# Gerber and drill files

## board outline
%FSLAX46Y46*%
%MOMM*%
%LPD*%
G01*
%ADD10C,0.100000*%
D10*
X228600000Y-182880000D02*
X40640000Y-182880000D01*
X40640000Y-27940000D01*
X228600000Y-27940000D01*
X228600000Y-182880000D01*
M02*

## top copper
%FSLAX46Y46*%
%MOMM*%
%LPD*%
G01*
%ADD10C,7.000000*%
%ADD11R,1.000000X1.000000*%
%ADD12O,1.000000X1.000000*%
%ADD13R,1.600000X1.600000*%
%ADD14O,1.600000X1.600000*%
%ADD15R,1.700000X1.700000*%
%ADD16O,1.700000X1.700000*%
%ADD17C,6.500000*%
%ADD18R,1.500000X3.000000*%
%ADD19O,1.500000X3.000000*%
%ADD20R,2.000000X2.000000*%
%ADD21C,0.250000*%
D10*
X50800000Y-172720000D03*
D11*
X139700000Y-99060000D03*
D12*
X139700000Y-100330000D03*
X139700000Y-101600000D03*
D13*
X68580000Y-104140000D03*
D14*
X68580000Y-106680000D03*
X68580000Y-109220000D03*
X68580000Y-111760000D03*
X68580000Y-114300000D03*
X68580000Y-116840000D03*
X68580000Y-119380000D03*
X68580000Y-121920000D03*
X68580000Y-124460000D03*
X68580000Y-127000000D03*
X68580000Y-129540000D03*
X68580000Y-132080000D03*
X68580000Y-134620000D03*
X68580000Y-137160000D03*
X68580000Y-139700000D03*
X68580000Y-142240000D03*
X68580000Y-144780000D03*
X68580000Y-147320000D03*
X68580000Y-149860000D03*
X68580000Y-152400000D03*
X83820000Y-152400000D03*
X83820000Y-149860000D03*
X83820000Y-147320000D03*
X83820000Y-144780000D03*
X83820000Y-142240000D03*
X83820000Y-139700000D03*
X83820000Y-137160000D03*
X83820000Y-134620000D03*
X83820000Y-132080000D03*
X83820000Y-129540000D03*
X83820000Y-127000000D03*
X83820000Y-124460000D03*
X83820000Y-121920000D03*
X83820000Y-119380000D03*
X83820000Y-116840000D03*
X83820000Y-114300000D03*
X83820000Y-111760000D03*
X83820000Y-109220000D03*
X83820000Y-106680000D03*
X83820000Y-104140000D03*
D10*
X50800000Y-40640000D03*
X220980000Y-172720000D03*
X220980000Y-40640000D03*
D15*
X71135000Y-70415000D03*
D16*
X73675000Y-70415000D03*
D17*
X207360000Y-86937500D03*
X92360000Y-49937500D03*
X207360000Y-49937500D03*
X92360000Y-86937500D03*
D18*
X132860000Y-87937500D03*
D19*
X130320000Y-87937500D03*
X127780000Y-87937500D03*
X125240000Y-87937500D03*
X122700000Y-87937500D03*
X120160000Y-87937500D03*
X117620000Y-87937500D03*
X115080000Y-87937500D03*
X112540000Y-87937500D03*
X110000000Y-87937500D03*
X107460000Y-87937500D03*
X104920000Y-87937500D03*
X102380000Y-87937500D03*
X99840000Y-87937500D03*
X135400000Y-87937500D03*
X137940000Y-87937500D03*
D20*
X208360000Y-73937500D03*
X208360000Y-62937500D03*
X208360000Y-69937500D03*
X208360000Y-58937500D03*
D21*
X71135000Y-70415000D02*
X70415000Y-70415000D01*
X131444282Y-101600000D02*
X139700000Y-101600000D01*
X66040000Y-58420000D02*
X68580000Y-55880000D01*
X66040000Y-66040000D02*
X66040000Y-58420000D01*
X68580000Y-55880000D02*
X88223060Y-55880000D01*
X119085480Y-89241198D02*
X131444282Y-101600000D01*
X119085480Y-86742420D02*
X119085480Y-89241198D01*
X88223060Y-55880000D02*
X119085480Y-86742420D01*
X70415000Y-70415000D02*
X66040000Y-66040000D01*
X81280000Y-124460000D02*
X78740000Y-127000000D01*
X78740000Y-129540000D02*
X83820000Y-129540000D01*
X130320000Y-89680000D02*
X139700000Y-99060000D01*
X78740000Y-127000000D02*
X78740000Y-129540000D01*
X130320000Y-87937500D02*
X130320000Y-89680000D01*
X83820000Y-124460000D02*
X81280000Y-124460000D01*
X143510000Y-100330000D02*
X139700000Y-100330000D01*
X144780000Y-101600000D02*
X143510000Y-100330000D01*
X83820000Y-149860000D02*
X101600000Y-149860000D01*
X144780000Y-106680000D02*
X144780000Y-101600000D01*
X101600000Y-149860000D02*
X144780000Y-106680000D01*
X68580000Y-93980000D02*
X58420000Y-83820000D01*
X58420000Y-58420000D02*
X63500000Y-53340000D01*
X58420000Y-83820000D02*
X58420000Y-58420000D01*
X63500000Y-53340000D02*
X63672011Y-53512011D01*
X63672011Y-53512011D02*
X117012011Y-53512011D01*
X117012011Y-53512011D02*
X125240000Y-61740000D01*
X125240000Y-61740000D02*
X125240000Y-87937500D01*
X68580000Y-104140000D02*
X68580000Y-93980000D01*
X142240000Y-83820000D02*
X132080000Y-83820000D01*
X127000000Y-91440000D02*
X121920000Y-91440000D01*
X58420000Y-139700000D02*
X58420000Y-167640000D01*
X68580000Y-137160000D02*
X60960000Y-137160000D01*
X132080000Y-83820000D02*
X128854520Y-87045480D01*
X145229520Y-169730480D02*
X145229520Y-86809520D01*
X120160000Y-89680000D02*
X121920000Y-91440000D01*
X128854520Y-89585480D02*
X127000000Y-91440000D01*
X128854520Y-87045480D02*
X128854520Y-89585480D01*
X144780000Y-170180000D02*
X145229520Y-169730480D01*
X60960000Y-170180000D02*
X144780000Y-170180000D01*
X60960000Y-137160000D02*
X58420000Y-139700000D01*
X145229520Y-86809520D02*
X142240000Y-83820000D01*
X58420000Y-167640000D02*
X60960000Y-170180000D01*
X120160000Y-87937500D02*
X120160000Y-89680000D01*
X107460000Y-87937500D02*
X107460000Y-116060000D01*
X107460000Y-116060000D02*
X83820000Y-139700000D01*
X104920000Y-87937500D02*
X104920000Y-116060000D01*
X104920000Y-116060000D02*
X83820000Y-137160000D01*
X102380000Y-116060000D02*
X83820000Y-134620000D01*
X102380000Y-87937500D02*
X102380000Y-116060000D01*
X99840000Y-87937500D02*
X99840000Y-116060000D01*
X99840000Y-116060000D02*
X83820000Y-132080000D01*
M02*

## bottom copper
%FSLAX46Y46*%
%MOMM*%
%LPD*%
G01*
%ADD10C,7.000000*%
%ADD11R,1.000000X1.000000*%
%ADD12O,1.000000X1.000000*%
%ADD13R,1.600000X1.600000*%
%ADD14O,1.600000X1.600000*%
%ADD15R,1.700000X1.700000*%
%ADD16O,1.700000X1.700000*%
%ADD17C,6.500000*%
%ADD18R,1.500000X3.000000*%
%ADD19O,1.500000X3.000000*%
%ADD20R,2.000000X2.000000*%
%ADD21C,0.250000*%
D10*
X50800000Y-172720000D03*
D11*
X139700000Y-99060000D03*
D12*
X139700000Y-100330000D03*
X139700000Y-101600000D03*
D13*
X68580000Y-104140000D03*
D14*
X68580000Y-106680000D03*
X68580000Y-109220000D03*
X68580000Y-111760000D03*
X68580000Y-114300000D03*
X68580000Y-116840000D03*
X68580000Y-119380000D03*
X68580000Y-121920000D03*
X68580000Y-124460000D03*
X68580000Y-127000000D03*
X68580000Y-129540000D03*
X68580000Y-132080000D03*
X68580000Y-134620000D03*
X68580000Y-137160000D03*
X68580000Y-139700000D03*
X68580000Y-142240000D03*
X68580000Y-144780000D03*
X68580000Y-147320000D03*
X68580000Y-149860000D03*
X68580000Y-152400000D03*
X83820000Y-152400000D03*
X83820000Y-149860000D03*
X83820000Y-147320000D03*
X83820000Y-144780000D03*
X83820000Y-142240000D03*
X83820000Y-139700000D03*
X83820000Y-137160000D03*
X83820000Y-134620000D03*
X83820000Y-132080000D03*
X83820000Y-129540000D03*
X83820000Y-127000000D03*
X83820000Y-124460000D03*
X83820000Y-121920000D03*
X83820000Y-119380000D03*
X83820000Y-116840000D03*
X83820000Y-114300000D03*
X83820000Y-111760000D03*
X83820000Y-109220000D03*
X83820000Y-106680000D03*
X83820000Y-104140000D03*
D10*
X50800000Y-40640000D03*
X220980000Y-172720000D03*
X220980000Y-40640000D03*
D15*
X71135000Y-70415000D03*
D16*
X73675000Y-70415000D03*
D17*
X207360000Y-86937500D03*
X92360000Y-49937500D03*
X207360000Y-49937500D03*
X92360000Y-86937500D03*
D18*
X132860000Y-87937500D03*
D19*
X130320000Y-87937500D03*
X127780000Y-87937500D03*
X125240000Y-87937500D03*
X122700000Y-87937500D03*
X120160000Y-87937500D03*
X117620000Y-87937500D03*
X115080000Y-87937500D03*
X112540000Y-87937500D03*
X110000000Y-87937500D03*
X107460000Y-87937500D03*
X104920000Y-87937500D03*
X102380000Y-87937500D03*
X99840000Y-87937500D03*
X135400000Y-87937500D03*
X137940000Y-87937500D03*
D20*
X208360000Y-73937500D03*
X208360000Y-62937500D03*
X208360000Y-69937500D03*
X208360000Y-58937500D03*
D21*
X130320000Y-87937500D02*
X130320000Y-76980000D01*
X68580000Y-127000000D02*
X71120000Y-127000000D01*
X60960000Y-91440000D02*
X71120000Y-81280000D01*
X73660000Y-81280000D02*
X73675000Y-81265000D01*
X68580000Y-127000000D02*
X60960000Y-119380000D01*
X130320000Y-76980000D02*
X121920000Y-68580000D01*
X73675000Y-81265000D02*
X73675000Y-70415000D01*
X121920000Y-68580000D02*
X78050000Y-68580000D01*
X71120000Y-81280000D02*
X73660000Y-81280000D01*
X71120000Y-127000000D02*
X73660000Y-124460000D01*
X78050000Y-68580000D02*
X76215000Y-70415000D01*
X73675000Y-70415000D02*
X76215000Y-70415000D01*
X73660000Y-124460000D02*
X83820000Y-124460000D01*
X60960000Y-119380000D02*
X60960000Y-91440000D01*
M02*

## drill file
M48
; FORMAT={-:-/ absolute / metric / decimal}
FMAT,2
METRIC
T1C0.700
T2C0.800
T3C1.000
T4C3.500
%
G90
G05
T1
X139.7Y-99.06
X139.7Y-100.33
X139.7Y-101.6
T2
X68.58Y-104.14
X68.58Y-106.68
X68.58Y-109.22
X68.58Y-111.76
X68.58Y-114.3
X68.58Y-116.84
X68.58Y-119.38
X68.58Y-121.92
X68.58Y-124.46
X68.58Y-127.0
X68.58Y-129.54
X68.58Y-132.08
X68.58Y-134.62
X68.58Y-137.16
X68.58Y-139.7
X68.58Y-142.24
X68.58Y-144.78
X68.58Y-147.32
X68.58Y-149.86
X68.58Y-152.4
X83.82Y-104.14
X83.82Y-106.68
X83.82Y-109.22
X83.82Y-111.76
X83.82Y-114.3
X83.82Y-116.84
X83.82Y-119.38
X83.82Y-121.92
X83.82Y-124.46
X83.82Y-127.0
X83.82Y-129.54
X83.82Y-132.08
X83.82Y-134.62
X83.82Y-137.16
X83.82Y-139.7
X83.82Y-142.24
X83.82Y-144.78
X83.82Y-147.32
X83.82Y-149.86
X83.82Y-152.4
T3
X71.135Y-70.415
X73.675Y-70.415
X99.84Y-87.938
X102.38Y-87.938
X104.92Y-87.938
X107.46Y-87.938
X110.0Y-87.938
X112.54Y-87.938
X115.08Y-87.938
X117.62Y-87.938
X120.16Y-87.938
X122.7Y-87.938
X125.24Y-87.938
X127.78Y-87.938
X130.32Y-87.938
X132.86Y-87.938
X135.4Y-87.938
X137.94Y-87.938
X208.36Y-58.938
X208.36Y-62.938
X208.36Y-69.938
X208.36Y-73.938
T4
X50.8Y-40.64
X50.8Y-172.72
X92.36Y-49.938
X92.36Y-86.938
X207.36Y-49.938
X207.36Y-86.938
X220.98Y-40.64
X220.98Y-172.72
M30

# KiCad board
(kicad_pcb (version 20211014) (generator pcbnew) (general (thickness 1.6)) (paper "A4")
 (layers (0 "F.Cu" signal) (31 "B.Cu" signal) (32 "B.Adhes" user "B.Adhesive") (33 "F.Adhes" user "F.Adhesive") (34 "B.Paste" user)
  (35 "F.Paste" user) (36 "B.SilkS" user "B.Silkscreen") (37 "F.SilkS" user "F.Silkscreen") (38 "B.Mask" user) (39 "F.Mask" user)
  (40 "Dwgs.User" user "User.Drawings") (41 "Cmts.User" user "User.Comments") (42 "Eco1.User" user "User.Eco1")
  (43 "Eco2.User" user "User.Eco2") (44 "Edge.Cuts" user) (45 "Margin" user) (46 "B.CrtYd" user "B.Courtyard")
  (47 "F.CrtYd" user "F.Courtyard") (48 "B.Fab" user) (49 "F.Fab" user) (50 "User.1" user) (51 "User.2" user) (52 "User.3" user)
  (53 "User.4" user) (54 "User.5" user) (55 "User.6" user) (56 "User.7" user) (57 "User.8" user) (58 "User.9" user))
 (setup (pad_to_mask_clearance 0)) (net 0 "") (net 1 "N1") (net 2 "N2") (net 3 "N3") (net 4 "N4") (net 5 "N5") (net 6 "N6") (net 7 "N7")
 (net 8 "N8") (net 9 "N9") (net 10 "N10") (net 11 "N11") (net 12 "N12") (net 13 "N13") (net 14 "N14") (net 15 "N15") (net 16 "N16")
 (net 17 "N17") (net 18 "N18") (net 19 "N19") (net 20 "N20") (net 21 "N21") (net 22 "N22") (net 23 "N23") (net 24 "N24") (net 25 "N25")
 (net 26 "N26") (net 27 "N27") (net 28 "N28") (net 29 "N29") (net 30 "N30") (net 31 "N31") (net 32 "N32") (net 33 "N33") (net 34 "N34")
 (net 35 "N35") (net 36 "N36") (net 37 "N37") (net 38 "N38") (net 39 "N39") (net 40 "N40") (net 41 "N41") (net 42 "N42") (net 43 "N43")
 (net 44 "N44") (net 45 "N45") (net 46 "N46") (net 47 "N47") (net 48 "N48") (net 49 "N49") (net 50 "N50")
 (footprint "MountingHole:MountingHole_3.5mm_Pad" (layer "F.Cu") (at 50.8 172.72)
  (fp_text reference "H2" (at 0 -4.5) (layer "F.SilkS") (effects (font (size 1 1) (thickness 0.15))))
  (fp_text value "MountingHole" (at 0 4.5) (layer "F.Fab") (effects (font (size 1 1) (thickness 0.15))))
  (pad "1" thru_hole circle (at 0 0) (size 7 7) (drill 3.5) (layers *.Cu *.Mask)))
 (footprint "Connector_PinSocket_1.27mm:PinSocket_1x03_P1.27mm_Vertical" (layer "F.Cu") (at 139.7 99.06)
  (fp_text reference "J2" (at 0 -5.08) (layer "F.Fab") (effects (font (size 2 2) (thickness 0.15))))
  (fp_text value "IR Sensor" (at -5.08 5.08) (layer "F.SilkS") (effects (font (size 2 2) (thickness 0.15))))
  (pad "1" thru_hole rect (at 0 0) (size 1 1) (drill 0.7) (layers *.Cu *.Mask) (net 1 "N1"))
  (pad "2" thru_hole oval (at 0 1.27) (size 1 1) (drill 0.7) (layers *.Cu *.Mask) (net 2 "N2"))
  (pad "3" thru_hole oval (at 0 2.54) (size 1 1) (drill 0.7) (layers *.Cu *.Mask) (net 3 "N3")))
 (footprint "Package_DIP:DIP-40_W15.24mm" (layer "F.Cu") (at 68.58 104.14)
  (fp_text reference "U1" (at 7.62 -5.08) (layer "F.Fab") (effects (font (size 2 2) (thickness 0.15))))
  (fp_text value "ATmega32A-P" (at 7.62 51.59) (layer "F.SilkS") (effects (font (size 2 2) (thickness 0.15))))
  (pad "1" thru_hole rect (at 0 0) (size 1.6 1.6) (drill 0.8) (layers *.Cu *.Mask) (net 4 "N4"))
  (pad "2" thru_hole oval (at 0 2.54) (size 1.6 1.6) (drill 0.8) (layers *.Cu *.Mask) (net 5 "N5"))
  (pad "3" thru_hole oval (at 0 5.08) (size 1.6 1.6) (drill 0.8) (layers *.Cu *.Mask) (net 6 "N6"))
  (pad "4" thru_hole oval (at 0 7.62) (size 1.6 1.6) (drill 0.8) (layers *.Cu *.Mask) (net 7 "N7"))
  (pad "5" thru_hole oval (at 0 10.16) (size 1.6 1.6) (drill 0.8) (layers *.Cu *.Mask) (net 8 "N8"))
  (pad "6" thru_hole oval (at 0 12.7) (size 1.6 1.6) (drill 0.8) (layers *.Cu *.Mask) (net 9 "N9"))
  (pad "7" thru_hole oval (at 0 15.24) (size 1.6 1.6) (drill 0.8) (layers *.Cu *.Mask) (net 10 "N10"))
  (pad "8" thru_hole oval (at 0 17.78) (size 1.6 1.6) (drill 0.8) (layers *.Cu *.Mask) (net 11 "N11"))
  (pad "9" thru_hole oval (at 0 20.32) (size 1.6 1.6) (drill 0.8) (layers *.Cu *.Mask) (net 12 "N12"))
  (pad "10" thru_hole oval (at 0 22.86) (size 1.6 1.6) (drill 0.8) (layers *.Cu *.Mask) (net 1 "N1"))
  (pad "11" thru_hole oval (at 0 25.4) (size 1.6 1.6) (drill 0.8) (layers *.Cu *.Mask) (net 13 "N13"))
  (pad "12" thru_hole oval (at 0 27.94) (size 1.6 1.6) (drill 0.8) (layers *.Cu *.Mask) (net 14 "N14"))
  (pad "13" thru_hole oval (at 0 30.48) (size 1.6 1.6) (drill 0.8) (layers *.Cu *.Mask) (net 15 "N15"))
  (pad "14" thru_hole oval (at 0 33.02) (size 1.6 1.6) (drill 0.8) (layers *.Cu *.Mask) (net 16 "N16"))
  (pad "15" thru_hole oval (at 0 35.56) (size 1.6 1.6) (drill 0.8) (layers *.Cu *.Mask) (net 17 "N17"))
  (pad "16" thru_hole oval (at 0 38.1) (size 1.6 1.6) (drill 0.8) (layers *.Cu *.Mask) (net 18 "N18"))
  (pad "17" thru_hole oval (at 0 40.64) (size 1.6 1.6) (drill 0.8) (layers *.Cu *.Mask) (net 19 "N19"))
  (pad "18" thru_hole oval (at 0 43.18) (size 1.6 1.6) (drill 0.8) (layers *.Cu *.Mask) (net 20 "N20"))
  (pad "19" thru_hole oval (at 0 45.72) (size 1.6 1.6) (drill 0.8) (layers *.Cu *.Mask) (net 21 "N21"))
  (pad "20" thru_hole oval (at 0 48.26) (size 1.6 1.6) (drill 0.8) (layers *.Cu *.Mask) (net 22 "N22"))
  (pad "21" thru_hole oval (at 15.24 48.26) (size 1.6 1.6) (drill 0.8) (layers *.Cu *.Mask) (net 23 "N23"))
  (pad "22" thru_hole oval (at 15.24 45.72) (size 1.6 1.6) (drill 0.8) (layers *.Cu *.Mask) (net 2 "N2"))
  (pad "23" thru_hole oval (at 15.24 43.18) (size 1.6 1.6) (drill 0.8) (layers *.Cu *.Mask) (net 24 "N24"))
  (pad "24" thru_hole oval (at 15.24 40.64) (size 1.6 1.6) (drill 0.8) (layers *.Cu *.Mask) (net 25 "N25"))
  (pad "25" thru_hole oval (at 15.24 38.1) (size 1.6 1.6) (drill 0.8) (layers *.Cu *.Mask) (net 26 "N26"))
  (pad "26" thru_hole oval (at 15.24 35.56) (size 1.6 1.6) (drill 0.8) (layers *.Cu *.Mask) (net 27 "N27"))
  (pad "27" thru_hole oval (at 15.24 33.02) (size 1.6 1.6) (drill 0.8) (layers *.Cu *.Mask) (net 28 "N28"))
  (pad "28" thru_hole oval (at 15.24 30.48) (size 1.6 1.6) (drill 0.8) (layers *.Cu *.Mask) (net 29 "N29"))
  (pad "29" thru_hole oval (at 15.24 27.94) (size 1.6 1.6) (drill 0.8) (layers *.Cu *.Mask) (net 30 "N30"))
  (pad "30" thru_hole oval (at 15.24 25.4) (size 1.6 1.6) (drill 0.8) (layers *.Cu *.Mask) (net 1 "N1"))
  (pad "31" thru_hole oval (at 15.24 22.86) (size 1.6 1.6) (drill 0.8) (layers *.Cu *.Mask) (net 13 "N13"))
  (pad "32" thru_hole oval (at 15.24 20.32) (size 1.6 1.6) (drill 0.8) (layers *.Cu *.Mask) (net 1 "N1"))
  (pad "33" thru_hole oval (at 15.24 17.78) (size 1.6 1.6) (drill 0.8) (layers *.Cu *.Mask) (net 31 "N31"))
  (pad "34" thru_hole oval (at 15.24 15.24) (size 1.6 1.6) (drill 0.8) (layers *.Cu *.Mask) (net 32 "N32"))
  (pad "35" thru_hole oval (at 15.24 12.7) (size 1.6 1.6) (drill 0.8) (layers *.Cu *.Mask) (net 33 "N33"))
  (pad "36" thru_hole oval (at 15.24 10.16) (size 1.6 1.6) (drill 0.8) (layers *.Cu *.Mask) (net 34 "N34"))
  (pad "37" thru_hole oval (at 15.24 7.62) (size 1.6 1.6) (drill 0.8) (layers *.Cu *.Mask) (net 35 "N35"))
  (pad "38" thru_hole oval (at 15.24 5.08) (size 1.6 1.6) (drill 0.8) (layers *.Cu *.Mask) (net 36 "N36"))
  (pad "39" thru_hole oval (at 15.24 2.54) (size 1.6 1.6) (drill 0.8) (layers *.Cu *.Mask) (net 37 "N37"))
  (pad "40" thru_hole oval (at 15.24 0) (size 1.6 1.6) (drill 0.8) (layers *.Cu *.Mask) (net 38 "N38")))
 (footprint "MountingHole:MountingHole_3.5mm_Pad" (layer "F.Cu") (at 50.8 40.64)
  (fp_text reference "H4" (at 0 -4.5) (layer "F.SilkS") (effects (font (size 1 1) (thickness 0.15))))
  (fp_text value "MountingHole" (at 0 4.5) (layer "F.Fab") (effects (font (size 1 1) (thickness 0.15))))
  (pad "1" thru_hole circle (at 0 0) (size 7 7) (drill 3.5) (layers *.Cu *.Mask)))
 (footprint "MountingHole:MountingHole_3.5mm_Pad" (layer "F.Cu") (at 220.98 172.72)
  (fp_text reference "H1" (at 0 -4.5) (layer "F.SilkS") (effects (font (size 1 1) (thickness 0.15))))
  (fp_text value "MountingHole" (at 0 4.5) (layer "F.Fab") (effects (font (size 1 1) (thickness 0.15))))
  (pad "1" thru_hole circle (at 0 0) (size 7 7) (drill 3.5) (layers *.Cu *.Mask)))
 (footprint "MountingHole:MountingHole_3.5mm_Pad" (layer "F.Cu") (at 220.98 40.64)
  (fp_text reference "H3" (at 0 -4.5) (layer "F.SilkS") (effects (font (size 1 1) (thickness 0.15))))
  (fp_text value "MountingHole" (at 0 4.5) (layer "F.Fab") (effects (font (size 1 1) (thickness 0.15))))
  (pad "1" thru_hole circle (at 0 0) (size 7 7) (drill 3.5) (layers *.Cu *.Mask)))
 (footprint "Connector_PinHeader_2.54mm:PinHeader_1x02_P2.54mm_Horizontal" (layer "F.Cu") (at 71.135 70.415 90)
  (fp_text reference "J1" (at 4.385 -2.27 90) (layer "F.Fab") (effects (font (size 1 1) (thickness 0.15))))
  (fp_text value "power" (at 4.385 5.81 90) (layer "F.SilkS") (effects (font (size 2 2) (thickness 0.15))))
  (pad "1" thru_hole rect (at 0 0 90) (size 1.7 1.7) (drill 1) (layers *.Cu *.Mask) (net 3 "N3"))
  (pad "2" thru_hole oval (at 0 2.54 90) (size 1.7 1.7) (drill 1) (layers *.Cu *.Mask) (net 1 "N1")))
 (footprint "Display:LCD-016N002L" (layer "F.Cu") (at 132.86 87.9375 180)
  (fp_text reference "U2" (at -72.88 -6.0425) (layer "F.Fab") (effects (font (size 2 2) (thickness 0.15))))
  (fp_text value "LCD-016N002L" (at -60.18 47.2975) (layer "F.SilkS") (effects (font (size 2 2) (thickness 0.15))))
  (pad "" thru_hole circle (at -74.5 1) (size 6.5 6.5) (drill 3.5) (layers *.Cu *.Mask))
  (pad "" thru_hole circle (at 40.5 38) (size 6.5 6.5) (drill 3.5) (layers *.Cu *.Mask))
  (pad "" thru_hole circle (at -74.5 38) (size 6.5 6.5) (drill 3.5) (layers *.Cu *.Mask))
  (pad "" thru_hole circle (at 40.5 1) (size 6.5 6.5) (drill 3.5) (layers *.Cu *.Mask))
  (pad "1" thru_hole rect (at 0 0) (size 1.5 3) (drill 1) (layers *.Cu *.Mask) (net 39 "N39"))
  (pad "2" thru_hole oval (at 2.54 0) (size 1.5 3) (drill 1) (layers *.Cu *.Mask) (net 1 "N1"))
  (pad "3" thru_hole oval (at 5.08 0) (size 1.5 3) (drill 1) (layers *.Cu *.Mask) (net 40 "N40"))
  (pad "4" thru_hole oval (at 7.62 0) (size 1.5 3) (drill 1) (layers *.Cu *.Mask) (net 4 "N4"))
  (pad "5" thru_hole oval (at 10.16 0) (size 1.5 3) (drill 1) (layers *.Cu *.Mask) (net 39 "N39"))
  (pad "6" thru_hole oval (at 12.7 0) (size 1.5 3) (drill 1) (layers *.Cu *.Mask) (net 16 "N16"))
  (pad "7" thru_hole oval (at 15.24 0) (size 1.5 3) (drill 1) (layers *.Cu *.Mask) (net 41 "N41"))
  (pad "8" thru_hole oval (at 17.78 0) (size 1.5 3) (drill 1) (layers *.Cu *.Mask) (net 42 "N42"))
  (pad "9" thru_hole oval (at 20.32 0) (size 1.5 3) (drill 1) (layers *.Cu *.Mask) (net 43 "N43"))
  (pad "10" thru_hole oval (at 22.86 0) (size 1.5 3) (drill 1) (layers *.Cu *.Mask) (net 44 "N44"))
  (pad "11" thru_hole oval (at 25.4 0) (size 1.5 3) (drill 1) (layers *.Cu *.Mask) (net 27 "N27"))
  (pad "12" thru_hole oval (at 27.94 0) (size 1.5 3) (drill 1) (layers *.Cu *.Mask) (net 28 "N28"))
  (pad "13" thru_hole oval (at 30.48 0) (size 1.5 3) (drill 1) (layers *.Cu *.Mask) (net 29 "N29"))
  (pad "14" thru_hole oval (at 33.02 0) (size 1.5 3) (drill 1) (layers *.Cu *.Mask) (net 30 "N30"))
  (pad "15" thru_hole oval (at -2.54 0) (size 1.5 3) (drill 1) (layers *.Cu *.Mask) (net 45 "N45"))
  (pad "16" thru_hole oval (at -5.08 0) (size 1.5 3) (drill 1) (layers *.Cu *.Mask) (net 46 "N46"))
  (pad "A1" thru_hole rect (at -75.5 14) (size 2 2) (drill 1) (layers *.Cu *.Mask) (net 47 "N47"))
  (pad "A2" thru_hole rect (at -75.5 25) (size 2 2) (drill 1) (layers *.Cu *.Mask) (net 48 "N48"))
  (pad "K1" thru_hole rect (at -75.5 18) (size 2 2) (drill 1) (layers *.Cu *.Mask) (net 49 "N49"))
  (pad "K2" thru_hole rect (at -75.5 29) (size 2 2) (drill 1) (layers *.Cu *.Mask) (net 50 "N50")))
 (gr_poly (pts (xy 228.6 182.88) (xy 40.64 182.88) (xy 40.64 27.94) (xy 228.6 27.94)) (layer "Edge.Cuts") (width 0.1) (fill none))
 (segment (start 71.135 70.415) (end 70.415 70.415) (width 0.25) (layer "F.Cu") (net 3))
 (segment (start 131.444282 101.6) (end 139.7 101.6) (width 0.25) (layer "F.Cu") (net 3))
 (segment (start 66.04 58.42) (end 68.58 55.88) (width 0.25) (layer "F.Cu") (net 3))
 (segment (start 66.04 66.04) (end 66.04 58.42) (width 0.25) (layer "F.Cu") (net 3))
 (segment (start 68.58 55.88) (end 88.22306 55.88) (width 0.25) (layer "F.Cu") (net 3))
 (segment (start 119.08548 89.241198) (end 131.444282 101.6) (width 0.25) (layer "F.Cu") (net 3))
 (segment (start 119.08548 86.74242) (end 119.08548 89.241198) (width 0.25) (layer "F.Cu") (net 3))
 (segment (start 88.22306 55.88) (end 119.08548 86.74242) (width 0.25) (layer "F.Cu") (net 3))
 (segment (start 70.415 70.415) (end 66.04 66.04) (width 0.25) (layer "F.Cu") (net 3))
 (segment (start 81.28 124.46) (end 78.74 127) (width 0.25) (layer "F.Cu") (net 1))
 (segment (start 78.74 129.54) (end 83.82 129.54) (width 0.25) (layer "F.Cu") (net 1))
 (segment (start 130.32 89.68) (end 139.7 99.06) (width 0.25) (layer "F.Cu") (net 1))
 (segment (start 78.74 127) (end 78.74 129.54) (width 0.25) (layer "F.Cu") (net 1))
 (segment (start 130.32 87.9375) (end 130.32 89.68) (width 0.25) (layer "F.Cu") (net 1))
 (segment (start 83.82 124.46) (end 81.28 124.46) (width 0.25) (layer "F.Cu") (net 1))
 (segment (start 130.32 87.9375) (end 130.32 76.98) (width 0.25) (layer "B.Cu") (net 1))
 (segment (start 68.58 127) (end 71.12 127) (width 0.25) (layer "B.Cu") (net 1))
 (segment (start 60.96 91.44) (end 71.12 81.28) (width 0.25) (layer "B.Cu") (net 1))
 (segment (start 73.66 81.28) (end 73.675 81.265) (width 0.25) (layer "B.Cu") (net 1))
 (segment (start 68.58 127) (end 60.96 119.38) (width 0.25) (layer "B.Cu") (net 1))
 (segment (start 130.32 76.98) (end 121.92 68.58) (width 0.25) (layer "B.Cu") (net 1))
 (segment (start 73.675 81.265) (end 73.675 70.415) (width 0.25) (layer "B.Cu") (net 1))
 (segment (start 121.92 68.58) (end 78.05 68.58) (width 0.25) (layer "B.Cu") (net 1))
 (segment (start 71.12 81.28) (end 73.66 81.28) (width 0.25) (layer "B.Cu") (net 1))
 (segment (start 71.12 127) (end 73.66 124.46) (width 0.25) (layer "B.Cu") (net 1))
 (segment (start 78.05 68.58) (end 76.215 70.415) (width 0.25) (layer "B.Cu") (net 1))
 (segment (start 73.675 70.415) (end 76.215 70.415) (width 0.25) (layer "B.Cu") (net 1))
 (segment (start 73.66 124.46) (end 83.82 124.46) (width 0.25) (layer "B.Cu") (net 1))
 (segment (start 60.96 119.38) (end 60.96 91.44) (width 0.25) (layer "B.Cu") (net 1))
 (segment (start 143.51 100.33) (end 139.7 100.33) (width 0.25) (layer "F.Cu") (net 2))
 (segment (start 144.78 101.6) (end 143.51 100.33) (width 0.25) (layer "F.Cu") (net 2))
 (segment (start 83.82 149.86) (end 101.6 149.86) (width 0.25) (layer "F.Cu") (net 2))
 (segment (start 144.78 106.68) (end 144.78 101.6) (width 0.25) (layer "F.Cu") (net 2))
 (segment (start 101.6 149.86) (end 144.78 106.68) (width 0.25) (layer "F.Cu") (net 2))
 (segment (start 68.58 93.98) (end 58.42 83.82) (width 0.25) (layer "F.Cu") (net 4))
 (segment (start 58.42 58.42) (end 63.5 53.34) (width 0.25) (layer "F.Cu") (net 4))
 (segment (start 58.42 83.82) (end 58.42 58.42) (width 0.25) (layer "F.Cu") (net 4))
 (segment (start 63.5 53.34) (end 63.672011 53.512011) (width 0.25) (layer "F.Cu") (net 4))
 (segment (start 63.672011 53.512011) (end 117.012011 53.512011) (width 0.25) (layer "F.Cu") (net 4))
 (segment (start 117.012011 53.512011) (end 125.24 61.74) (width 0.25) (layer "F.Cu") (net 4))
 (segment (start 125.24 61.74) (end 125.24 87.9375) (width 0.25) (layer "F.Cu") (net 4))
 (segment (start 68.58 104.14) (end 68.58 93.98) (width 0.25) (layer "F.Cu") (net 4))
 (segment (start 142.24 83.82) (end 132.08 83.82) (width 0.25) (layer "F.Cu") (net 16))
 (segment (start 127 91.44) (end 121.92 91.44) (width 0.25) (layer "F.Cu") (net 16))
 (segment (start 58.42 139.7) (end 58.42 167.64) (width 0.25) (layer "F.Cu") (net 16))
 (segment (start 68.58 137.16) (end 60.96 137.16) (width 0.25) (layer "F.Cu") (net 16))
 (segment (start 132.08 83.82) (end 128.85452 87.04548) (width 0.25) (layer "F.Cu") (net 16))
 (segment (start 145.22952 169.73048) (end 145.22952 86.80952) (width 0.25) (layer "F.Cu") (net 16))
 (segment (start 120.16 89.68) (end 121.92 91.44) (width 0.25) (layer "F.Cu") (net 16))
 (segment (start 128.85452 89.58548) (end 127 91.44) (width 0.25) (layer "F.Cu") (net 16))
 (segment (start 128.85452 87.04548) (end 128.85452 89.58548) (width 0.25) (layer "F.Cu") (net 16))
 (segment (start 144.78 170.18) (end 145.22952 169.73048) (width 0.25) (layer "F.Cu") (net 16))
 (segment (start 60.96 170.18) (end 144.78 170.18) (width 0.25) (layer "F.Cu") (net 16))
 (segment (start 60.96 137.16) (end 58.42 139.7) (width 0.25) (layer "F.Cu") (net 16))
 (segment (start 145.22952 86.80952) (end 142.24 83.82) (width 0.25) (layer "F.Cu") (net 16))
 (segment (start 58.42 167.64) (end 60.96 170.18) (width 0.25) (layer "F.Cu") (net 16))
 (segment (start 120.16 87.9375) (end 120.16 89.68) (width 0.25) (layer "F.Cu") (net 16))
 (segment (start 107.46 87.9375) (end 107.46 116.06) (width 0.25) (layer "F.Cu") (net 27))
 (segment (start 107.46 116.06) (end 83.82 139.7) (width 0.25) (layer "F.Cu") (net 27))
 (segment (start 104.92 87.9375) (end 104.92 116.06) (width 0.25) (layer "F.Cu") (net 28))
 (segment (start 104.92 116.06) (end 83.82 137.16) (width 0.25) (layer "F.Cu") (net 28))
 (segment (start 102.38 116.06) (end 83.82 134.62) (width 0.25) (layer "F.Cu") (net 29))
 (segment (start 102.38 87.9375) (end 102.38 116.06) (width 0.25) (layer "F.Cu") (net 29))
 (segment (start 99.84 87.9375) (end 99.84 116.06) (width 0.25) (layer "F.Cu") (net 30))
 (segment (start 99.84 116.06) (end 83.82 132.08) (width 0.25) (layer "F.Cu") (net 30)))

